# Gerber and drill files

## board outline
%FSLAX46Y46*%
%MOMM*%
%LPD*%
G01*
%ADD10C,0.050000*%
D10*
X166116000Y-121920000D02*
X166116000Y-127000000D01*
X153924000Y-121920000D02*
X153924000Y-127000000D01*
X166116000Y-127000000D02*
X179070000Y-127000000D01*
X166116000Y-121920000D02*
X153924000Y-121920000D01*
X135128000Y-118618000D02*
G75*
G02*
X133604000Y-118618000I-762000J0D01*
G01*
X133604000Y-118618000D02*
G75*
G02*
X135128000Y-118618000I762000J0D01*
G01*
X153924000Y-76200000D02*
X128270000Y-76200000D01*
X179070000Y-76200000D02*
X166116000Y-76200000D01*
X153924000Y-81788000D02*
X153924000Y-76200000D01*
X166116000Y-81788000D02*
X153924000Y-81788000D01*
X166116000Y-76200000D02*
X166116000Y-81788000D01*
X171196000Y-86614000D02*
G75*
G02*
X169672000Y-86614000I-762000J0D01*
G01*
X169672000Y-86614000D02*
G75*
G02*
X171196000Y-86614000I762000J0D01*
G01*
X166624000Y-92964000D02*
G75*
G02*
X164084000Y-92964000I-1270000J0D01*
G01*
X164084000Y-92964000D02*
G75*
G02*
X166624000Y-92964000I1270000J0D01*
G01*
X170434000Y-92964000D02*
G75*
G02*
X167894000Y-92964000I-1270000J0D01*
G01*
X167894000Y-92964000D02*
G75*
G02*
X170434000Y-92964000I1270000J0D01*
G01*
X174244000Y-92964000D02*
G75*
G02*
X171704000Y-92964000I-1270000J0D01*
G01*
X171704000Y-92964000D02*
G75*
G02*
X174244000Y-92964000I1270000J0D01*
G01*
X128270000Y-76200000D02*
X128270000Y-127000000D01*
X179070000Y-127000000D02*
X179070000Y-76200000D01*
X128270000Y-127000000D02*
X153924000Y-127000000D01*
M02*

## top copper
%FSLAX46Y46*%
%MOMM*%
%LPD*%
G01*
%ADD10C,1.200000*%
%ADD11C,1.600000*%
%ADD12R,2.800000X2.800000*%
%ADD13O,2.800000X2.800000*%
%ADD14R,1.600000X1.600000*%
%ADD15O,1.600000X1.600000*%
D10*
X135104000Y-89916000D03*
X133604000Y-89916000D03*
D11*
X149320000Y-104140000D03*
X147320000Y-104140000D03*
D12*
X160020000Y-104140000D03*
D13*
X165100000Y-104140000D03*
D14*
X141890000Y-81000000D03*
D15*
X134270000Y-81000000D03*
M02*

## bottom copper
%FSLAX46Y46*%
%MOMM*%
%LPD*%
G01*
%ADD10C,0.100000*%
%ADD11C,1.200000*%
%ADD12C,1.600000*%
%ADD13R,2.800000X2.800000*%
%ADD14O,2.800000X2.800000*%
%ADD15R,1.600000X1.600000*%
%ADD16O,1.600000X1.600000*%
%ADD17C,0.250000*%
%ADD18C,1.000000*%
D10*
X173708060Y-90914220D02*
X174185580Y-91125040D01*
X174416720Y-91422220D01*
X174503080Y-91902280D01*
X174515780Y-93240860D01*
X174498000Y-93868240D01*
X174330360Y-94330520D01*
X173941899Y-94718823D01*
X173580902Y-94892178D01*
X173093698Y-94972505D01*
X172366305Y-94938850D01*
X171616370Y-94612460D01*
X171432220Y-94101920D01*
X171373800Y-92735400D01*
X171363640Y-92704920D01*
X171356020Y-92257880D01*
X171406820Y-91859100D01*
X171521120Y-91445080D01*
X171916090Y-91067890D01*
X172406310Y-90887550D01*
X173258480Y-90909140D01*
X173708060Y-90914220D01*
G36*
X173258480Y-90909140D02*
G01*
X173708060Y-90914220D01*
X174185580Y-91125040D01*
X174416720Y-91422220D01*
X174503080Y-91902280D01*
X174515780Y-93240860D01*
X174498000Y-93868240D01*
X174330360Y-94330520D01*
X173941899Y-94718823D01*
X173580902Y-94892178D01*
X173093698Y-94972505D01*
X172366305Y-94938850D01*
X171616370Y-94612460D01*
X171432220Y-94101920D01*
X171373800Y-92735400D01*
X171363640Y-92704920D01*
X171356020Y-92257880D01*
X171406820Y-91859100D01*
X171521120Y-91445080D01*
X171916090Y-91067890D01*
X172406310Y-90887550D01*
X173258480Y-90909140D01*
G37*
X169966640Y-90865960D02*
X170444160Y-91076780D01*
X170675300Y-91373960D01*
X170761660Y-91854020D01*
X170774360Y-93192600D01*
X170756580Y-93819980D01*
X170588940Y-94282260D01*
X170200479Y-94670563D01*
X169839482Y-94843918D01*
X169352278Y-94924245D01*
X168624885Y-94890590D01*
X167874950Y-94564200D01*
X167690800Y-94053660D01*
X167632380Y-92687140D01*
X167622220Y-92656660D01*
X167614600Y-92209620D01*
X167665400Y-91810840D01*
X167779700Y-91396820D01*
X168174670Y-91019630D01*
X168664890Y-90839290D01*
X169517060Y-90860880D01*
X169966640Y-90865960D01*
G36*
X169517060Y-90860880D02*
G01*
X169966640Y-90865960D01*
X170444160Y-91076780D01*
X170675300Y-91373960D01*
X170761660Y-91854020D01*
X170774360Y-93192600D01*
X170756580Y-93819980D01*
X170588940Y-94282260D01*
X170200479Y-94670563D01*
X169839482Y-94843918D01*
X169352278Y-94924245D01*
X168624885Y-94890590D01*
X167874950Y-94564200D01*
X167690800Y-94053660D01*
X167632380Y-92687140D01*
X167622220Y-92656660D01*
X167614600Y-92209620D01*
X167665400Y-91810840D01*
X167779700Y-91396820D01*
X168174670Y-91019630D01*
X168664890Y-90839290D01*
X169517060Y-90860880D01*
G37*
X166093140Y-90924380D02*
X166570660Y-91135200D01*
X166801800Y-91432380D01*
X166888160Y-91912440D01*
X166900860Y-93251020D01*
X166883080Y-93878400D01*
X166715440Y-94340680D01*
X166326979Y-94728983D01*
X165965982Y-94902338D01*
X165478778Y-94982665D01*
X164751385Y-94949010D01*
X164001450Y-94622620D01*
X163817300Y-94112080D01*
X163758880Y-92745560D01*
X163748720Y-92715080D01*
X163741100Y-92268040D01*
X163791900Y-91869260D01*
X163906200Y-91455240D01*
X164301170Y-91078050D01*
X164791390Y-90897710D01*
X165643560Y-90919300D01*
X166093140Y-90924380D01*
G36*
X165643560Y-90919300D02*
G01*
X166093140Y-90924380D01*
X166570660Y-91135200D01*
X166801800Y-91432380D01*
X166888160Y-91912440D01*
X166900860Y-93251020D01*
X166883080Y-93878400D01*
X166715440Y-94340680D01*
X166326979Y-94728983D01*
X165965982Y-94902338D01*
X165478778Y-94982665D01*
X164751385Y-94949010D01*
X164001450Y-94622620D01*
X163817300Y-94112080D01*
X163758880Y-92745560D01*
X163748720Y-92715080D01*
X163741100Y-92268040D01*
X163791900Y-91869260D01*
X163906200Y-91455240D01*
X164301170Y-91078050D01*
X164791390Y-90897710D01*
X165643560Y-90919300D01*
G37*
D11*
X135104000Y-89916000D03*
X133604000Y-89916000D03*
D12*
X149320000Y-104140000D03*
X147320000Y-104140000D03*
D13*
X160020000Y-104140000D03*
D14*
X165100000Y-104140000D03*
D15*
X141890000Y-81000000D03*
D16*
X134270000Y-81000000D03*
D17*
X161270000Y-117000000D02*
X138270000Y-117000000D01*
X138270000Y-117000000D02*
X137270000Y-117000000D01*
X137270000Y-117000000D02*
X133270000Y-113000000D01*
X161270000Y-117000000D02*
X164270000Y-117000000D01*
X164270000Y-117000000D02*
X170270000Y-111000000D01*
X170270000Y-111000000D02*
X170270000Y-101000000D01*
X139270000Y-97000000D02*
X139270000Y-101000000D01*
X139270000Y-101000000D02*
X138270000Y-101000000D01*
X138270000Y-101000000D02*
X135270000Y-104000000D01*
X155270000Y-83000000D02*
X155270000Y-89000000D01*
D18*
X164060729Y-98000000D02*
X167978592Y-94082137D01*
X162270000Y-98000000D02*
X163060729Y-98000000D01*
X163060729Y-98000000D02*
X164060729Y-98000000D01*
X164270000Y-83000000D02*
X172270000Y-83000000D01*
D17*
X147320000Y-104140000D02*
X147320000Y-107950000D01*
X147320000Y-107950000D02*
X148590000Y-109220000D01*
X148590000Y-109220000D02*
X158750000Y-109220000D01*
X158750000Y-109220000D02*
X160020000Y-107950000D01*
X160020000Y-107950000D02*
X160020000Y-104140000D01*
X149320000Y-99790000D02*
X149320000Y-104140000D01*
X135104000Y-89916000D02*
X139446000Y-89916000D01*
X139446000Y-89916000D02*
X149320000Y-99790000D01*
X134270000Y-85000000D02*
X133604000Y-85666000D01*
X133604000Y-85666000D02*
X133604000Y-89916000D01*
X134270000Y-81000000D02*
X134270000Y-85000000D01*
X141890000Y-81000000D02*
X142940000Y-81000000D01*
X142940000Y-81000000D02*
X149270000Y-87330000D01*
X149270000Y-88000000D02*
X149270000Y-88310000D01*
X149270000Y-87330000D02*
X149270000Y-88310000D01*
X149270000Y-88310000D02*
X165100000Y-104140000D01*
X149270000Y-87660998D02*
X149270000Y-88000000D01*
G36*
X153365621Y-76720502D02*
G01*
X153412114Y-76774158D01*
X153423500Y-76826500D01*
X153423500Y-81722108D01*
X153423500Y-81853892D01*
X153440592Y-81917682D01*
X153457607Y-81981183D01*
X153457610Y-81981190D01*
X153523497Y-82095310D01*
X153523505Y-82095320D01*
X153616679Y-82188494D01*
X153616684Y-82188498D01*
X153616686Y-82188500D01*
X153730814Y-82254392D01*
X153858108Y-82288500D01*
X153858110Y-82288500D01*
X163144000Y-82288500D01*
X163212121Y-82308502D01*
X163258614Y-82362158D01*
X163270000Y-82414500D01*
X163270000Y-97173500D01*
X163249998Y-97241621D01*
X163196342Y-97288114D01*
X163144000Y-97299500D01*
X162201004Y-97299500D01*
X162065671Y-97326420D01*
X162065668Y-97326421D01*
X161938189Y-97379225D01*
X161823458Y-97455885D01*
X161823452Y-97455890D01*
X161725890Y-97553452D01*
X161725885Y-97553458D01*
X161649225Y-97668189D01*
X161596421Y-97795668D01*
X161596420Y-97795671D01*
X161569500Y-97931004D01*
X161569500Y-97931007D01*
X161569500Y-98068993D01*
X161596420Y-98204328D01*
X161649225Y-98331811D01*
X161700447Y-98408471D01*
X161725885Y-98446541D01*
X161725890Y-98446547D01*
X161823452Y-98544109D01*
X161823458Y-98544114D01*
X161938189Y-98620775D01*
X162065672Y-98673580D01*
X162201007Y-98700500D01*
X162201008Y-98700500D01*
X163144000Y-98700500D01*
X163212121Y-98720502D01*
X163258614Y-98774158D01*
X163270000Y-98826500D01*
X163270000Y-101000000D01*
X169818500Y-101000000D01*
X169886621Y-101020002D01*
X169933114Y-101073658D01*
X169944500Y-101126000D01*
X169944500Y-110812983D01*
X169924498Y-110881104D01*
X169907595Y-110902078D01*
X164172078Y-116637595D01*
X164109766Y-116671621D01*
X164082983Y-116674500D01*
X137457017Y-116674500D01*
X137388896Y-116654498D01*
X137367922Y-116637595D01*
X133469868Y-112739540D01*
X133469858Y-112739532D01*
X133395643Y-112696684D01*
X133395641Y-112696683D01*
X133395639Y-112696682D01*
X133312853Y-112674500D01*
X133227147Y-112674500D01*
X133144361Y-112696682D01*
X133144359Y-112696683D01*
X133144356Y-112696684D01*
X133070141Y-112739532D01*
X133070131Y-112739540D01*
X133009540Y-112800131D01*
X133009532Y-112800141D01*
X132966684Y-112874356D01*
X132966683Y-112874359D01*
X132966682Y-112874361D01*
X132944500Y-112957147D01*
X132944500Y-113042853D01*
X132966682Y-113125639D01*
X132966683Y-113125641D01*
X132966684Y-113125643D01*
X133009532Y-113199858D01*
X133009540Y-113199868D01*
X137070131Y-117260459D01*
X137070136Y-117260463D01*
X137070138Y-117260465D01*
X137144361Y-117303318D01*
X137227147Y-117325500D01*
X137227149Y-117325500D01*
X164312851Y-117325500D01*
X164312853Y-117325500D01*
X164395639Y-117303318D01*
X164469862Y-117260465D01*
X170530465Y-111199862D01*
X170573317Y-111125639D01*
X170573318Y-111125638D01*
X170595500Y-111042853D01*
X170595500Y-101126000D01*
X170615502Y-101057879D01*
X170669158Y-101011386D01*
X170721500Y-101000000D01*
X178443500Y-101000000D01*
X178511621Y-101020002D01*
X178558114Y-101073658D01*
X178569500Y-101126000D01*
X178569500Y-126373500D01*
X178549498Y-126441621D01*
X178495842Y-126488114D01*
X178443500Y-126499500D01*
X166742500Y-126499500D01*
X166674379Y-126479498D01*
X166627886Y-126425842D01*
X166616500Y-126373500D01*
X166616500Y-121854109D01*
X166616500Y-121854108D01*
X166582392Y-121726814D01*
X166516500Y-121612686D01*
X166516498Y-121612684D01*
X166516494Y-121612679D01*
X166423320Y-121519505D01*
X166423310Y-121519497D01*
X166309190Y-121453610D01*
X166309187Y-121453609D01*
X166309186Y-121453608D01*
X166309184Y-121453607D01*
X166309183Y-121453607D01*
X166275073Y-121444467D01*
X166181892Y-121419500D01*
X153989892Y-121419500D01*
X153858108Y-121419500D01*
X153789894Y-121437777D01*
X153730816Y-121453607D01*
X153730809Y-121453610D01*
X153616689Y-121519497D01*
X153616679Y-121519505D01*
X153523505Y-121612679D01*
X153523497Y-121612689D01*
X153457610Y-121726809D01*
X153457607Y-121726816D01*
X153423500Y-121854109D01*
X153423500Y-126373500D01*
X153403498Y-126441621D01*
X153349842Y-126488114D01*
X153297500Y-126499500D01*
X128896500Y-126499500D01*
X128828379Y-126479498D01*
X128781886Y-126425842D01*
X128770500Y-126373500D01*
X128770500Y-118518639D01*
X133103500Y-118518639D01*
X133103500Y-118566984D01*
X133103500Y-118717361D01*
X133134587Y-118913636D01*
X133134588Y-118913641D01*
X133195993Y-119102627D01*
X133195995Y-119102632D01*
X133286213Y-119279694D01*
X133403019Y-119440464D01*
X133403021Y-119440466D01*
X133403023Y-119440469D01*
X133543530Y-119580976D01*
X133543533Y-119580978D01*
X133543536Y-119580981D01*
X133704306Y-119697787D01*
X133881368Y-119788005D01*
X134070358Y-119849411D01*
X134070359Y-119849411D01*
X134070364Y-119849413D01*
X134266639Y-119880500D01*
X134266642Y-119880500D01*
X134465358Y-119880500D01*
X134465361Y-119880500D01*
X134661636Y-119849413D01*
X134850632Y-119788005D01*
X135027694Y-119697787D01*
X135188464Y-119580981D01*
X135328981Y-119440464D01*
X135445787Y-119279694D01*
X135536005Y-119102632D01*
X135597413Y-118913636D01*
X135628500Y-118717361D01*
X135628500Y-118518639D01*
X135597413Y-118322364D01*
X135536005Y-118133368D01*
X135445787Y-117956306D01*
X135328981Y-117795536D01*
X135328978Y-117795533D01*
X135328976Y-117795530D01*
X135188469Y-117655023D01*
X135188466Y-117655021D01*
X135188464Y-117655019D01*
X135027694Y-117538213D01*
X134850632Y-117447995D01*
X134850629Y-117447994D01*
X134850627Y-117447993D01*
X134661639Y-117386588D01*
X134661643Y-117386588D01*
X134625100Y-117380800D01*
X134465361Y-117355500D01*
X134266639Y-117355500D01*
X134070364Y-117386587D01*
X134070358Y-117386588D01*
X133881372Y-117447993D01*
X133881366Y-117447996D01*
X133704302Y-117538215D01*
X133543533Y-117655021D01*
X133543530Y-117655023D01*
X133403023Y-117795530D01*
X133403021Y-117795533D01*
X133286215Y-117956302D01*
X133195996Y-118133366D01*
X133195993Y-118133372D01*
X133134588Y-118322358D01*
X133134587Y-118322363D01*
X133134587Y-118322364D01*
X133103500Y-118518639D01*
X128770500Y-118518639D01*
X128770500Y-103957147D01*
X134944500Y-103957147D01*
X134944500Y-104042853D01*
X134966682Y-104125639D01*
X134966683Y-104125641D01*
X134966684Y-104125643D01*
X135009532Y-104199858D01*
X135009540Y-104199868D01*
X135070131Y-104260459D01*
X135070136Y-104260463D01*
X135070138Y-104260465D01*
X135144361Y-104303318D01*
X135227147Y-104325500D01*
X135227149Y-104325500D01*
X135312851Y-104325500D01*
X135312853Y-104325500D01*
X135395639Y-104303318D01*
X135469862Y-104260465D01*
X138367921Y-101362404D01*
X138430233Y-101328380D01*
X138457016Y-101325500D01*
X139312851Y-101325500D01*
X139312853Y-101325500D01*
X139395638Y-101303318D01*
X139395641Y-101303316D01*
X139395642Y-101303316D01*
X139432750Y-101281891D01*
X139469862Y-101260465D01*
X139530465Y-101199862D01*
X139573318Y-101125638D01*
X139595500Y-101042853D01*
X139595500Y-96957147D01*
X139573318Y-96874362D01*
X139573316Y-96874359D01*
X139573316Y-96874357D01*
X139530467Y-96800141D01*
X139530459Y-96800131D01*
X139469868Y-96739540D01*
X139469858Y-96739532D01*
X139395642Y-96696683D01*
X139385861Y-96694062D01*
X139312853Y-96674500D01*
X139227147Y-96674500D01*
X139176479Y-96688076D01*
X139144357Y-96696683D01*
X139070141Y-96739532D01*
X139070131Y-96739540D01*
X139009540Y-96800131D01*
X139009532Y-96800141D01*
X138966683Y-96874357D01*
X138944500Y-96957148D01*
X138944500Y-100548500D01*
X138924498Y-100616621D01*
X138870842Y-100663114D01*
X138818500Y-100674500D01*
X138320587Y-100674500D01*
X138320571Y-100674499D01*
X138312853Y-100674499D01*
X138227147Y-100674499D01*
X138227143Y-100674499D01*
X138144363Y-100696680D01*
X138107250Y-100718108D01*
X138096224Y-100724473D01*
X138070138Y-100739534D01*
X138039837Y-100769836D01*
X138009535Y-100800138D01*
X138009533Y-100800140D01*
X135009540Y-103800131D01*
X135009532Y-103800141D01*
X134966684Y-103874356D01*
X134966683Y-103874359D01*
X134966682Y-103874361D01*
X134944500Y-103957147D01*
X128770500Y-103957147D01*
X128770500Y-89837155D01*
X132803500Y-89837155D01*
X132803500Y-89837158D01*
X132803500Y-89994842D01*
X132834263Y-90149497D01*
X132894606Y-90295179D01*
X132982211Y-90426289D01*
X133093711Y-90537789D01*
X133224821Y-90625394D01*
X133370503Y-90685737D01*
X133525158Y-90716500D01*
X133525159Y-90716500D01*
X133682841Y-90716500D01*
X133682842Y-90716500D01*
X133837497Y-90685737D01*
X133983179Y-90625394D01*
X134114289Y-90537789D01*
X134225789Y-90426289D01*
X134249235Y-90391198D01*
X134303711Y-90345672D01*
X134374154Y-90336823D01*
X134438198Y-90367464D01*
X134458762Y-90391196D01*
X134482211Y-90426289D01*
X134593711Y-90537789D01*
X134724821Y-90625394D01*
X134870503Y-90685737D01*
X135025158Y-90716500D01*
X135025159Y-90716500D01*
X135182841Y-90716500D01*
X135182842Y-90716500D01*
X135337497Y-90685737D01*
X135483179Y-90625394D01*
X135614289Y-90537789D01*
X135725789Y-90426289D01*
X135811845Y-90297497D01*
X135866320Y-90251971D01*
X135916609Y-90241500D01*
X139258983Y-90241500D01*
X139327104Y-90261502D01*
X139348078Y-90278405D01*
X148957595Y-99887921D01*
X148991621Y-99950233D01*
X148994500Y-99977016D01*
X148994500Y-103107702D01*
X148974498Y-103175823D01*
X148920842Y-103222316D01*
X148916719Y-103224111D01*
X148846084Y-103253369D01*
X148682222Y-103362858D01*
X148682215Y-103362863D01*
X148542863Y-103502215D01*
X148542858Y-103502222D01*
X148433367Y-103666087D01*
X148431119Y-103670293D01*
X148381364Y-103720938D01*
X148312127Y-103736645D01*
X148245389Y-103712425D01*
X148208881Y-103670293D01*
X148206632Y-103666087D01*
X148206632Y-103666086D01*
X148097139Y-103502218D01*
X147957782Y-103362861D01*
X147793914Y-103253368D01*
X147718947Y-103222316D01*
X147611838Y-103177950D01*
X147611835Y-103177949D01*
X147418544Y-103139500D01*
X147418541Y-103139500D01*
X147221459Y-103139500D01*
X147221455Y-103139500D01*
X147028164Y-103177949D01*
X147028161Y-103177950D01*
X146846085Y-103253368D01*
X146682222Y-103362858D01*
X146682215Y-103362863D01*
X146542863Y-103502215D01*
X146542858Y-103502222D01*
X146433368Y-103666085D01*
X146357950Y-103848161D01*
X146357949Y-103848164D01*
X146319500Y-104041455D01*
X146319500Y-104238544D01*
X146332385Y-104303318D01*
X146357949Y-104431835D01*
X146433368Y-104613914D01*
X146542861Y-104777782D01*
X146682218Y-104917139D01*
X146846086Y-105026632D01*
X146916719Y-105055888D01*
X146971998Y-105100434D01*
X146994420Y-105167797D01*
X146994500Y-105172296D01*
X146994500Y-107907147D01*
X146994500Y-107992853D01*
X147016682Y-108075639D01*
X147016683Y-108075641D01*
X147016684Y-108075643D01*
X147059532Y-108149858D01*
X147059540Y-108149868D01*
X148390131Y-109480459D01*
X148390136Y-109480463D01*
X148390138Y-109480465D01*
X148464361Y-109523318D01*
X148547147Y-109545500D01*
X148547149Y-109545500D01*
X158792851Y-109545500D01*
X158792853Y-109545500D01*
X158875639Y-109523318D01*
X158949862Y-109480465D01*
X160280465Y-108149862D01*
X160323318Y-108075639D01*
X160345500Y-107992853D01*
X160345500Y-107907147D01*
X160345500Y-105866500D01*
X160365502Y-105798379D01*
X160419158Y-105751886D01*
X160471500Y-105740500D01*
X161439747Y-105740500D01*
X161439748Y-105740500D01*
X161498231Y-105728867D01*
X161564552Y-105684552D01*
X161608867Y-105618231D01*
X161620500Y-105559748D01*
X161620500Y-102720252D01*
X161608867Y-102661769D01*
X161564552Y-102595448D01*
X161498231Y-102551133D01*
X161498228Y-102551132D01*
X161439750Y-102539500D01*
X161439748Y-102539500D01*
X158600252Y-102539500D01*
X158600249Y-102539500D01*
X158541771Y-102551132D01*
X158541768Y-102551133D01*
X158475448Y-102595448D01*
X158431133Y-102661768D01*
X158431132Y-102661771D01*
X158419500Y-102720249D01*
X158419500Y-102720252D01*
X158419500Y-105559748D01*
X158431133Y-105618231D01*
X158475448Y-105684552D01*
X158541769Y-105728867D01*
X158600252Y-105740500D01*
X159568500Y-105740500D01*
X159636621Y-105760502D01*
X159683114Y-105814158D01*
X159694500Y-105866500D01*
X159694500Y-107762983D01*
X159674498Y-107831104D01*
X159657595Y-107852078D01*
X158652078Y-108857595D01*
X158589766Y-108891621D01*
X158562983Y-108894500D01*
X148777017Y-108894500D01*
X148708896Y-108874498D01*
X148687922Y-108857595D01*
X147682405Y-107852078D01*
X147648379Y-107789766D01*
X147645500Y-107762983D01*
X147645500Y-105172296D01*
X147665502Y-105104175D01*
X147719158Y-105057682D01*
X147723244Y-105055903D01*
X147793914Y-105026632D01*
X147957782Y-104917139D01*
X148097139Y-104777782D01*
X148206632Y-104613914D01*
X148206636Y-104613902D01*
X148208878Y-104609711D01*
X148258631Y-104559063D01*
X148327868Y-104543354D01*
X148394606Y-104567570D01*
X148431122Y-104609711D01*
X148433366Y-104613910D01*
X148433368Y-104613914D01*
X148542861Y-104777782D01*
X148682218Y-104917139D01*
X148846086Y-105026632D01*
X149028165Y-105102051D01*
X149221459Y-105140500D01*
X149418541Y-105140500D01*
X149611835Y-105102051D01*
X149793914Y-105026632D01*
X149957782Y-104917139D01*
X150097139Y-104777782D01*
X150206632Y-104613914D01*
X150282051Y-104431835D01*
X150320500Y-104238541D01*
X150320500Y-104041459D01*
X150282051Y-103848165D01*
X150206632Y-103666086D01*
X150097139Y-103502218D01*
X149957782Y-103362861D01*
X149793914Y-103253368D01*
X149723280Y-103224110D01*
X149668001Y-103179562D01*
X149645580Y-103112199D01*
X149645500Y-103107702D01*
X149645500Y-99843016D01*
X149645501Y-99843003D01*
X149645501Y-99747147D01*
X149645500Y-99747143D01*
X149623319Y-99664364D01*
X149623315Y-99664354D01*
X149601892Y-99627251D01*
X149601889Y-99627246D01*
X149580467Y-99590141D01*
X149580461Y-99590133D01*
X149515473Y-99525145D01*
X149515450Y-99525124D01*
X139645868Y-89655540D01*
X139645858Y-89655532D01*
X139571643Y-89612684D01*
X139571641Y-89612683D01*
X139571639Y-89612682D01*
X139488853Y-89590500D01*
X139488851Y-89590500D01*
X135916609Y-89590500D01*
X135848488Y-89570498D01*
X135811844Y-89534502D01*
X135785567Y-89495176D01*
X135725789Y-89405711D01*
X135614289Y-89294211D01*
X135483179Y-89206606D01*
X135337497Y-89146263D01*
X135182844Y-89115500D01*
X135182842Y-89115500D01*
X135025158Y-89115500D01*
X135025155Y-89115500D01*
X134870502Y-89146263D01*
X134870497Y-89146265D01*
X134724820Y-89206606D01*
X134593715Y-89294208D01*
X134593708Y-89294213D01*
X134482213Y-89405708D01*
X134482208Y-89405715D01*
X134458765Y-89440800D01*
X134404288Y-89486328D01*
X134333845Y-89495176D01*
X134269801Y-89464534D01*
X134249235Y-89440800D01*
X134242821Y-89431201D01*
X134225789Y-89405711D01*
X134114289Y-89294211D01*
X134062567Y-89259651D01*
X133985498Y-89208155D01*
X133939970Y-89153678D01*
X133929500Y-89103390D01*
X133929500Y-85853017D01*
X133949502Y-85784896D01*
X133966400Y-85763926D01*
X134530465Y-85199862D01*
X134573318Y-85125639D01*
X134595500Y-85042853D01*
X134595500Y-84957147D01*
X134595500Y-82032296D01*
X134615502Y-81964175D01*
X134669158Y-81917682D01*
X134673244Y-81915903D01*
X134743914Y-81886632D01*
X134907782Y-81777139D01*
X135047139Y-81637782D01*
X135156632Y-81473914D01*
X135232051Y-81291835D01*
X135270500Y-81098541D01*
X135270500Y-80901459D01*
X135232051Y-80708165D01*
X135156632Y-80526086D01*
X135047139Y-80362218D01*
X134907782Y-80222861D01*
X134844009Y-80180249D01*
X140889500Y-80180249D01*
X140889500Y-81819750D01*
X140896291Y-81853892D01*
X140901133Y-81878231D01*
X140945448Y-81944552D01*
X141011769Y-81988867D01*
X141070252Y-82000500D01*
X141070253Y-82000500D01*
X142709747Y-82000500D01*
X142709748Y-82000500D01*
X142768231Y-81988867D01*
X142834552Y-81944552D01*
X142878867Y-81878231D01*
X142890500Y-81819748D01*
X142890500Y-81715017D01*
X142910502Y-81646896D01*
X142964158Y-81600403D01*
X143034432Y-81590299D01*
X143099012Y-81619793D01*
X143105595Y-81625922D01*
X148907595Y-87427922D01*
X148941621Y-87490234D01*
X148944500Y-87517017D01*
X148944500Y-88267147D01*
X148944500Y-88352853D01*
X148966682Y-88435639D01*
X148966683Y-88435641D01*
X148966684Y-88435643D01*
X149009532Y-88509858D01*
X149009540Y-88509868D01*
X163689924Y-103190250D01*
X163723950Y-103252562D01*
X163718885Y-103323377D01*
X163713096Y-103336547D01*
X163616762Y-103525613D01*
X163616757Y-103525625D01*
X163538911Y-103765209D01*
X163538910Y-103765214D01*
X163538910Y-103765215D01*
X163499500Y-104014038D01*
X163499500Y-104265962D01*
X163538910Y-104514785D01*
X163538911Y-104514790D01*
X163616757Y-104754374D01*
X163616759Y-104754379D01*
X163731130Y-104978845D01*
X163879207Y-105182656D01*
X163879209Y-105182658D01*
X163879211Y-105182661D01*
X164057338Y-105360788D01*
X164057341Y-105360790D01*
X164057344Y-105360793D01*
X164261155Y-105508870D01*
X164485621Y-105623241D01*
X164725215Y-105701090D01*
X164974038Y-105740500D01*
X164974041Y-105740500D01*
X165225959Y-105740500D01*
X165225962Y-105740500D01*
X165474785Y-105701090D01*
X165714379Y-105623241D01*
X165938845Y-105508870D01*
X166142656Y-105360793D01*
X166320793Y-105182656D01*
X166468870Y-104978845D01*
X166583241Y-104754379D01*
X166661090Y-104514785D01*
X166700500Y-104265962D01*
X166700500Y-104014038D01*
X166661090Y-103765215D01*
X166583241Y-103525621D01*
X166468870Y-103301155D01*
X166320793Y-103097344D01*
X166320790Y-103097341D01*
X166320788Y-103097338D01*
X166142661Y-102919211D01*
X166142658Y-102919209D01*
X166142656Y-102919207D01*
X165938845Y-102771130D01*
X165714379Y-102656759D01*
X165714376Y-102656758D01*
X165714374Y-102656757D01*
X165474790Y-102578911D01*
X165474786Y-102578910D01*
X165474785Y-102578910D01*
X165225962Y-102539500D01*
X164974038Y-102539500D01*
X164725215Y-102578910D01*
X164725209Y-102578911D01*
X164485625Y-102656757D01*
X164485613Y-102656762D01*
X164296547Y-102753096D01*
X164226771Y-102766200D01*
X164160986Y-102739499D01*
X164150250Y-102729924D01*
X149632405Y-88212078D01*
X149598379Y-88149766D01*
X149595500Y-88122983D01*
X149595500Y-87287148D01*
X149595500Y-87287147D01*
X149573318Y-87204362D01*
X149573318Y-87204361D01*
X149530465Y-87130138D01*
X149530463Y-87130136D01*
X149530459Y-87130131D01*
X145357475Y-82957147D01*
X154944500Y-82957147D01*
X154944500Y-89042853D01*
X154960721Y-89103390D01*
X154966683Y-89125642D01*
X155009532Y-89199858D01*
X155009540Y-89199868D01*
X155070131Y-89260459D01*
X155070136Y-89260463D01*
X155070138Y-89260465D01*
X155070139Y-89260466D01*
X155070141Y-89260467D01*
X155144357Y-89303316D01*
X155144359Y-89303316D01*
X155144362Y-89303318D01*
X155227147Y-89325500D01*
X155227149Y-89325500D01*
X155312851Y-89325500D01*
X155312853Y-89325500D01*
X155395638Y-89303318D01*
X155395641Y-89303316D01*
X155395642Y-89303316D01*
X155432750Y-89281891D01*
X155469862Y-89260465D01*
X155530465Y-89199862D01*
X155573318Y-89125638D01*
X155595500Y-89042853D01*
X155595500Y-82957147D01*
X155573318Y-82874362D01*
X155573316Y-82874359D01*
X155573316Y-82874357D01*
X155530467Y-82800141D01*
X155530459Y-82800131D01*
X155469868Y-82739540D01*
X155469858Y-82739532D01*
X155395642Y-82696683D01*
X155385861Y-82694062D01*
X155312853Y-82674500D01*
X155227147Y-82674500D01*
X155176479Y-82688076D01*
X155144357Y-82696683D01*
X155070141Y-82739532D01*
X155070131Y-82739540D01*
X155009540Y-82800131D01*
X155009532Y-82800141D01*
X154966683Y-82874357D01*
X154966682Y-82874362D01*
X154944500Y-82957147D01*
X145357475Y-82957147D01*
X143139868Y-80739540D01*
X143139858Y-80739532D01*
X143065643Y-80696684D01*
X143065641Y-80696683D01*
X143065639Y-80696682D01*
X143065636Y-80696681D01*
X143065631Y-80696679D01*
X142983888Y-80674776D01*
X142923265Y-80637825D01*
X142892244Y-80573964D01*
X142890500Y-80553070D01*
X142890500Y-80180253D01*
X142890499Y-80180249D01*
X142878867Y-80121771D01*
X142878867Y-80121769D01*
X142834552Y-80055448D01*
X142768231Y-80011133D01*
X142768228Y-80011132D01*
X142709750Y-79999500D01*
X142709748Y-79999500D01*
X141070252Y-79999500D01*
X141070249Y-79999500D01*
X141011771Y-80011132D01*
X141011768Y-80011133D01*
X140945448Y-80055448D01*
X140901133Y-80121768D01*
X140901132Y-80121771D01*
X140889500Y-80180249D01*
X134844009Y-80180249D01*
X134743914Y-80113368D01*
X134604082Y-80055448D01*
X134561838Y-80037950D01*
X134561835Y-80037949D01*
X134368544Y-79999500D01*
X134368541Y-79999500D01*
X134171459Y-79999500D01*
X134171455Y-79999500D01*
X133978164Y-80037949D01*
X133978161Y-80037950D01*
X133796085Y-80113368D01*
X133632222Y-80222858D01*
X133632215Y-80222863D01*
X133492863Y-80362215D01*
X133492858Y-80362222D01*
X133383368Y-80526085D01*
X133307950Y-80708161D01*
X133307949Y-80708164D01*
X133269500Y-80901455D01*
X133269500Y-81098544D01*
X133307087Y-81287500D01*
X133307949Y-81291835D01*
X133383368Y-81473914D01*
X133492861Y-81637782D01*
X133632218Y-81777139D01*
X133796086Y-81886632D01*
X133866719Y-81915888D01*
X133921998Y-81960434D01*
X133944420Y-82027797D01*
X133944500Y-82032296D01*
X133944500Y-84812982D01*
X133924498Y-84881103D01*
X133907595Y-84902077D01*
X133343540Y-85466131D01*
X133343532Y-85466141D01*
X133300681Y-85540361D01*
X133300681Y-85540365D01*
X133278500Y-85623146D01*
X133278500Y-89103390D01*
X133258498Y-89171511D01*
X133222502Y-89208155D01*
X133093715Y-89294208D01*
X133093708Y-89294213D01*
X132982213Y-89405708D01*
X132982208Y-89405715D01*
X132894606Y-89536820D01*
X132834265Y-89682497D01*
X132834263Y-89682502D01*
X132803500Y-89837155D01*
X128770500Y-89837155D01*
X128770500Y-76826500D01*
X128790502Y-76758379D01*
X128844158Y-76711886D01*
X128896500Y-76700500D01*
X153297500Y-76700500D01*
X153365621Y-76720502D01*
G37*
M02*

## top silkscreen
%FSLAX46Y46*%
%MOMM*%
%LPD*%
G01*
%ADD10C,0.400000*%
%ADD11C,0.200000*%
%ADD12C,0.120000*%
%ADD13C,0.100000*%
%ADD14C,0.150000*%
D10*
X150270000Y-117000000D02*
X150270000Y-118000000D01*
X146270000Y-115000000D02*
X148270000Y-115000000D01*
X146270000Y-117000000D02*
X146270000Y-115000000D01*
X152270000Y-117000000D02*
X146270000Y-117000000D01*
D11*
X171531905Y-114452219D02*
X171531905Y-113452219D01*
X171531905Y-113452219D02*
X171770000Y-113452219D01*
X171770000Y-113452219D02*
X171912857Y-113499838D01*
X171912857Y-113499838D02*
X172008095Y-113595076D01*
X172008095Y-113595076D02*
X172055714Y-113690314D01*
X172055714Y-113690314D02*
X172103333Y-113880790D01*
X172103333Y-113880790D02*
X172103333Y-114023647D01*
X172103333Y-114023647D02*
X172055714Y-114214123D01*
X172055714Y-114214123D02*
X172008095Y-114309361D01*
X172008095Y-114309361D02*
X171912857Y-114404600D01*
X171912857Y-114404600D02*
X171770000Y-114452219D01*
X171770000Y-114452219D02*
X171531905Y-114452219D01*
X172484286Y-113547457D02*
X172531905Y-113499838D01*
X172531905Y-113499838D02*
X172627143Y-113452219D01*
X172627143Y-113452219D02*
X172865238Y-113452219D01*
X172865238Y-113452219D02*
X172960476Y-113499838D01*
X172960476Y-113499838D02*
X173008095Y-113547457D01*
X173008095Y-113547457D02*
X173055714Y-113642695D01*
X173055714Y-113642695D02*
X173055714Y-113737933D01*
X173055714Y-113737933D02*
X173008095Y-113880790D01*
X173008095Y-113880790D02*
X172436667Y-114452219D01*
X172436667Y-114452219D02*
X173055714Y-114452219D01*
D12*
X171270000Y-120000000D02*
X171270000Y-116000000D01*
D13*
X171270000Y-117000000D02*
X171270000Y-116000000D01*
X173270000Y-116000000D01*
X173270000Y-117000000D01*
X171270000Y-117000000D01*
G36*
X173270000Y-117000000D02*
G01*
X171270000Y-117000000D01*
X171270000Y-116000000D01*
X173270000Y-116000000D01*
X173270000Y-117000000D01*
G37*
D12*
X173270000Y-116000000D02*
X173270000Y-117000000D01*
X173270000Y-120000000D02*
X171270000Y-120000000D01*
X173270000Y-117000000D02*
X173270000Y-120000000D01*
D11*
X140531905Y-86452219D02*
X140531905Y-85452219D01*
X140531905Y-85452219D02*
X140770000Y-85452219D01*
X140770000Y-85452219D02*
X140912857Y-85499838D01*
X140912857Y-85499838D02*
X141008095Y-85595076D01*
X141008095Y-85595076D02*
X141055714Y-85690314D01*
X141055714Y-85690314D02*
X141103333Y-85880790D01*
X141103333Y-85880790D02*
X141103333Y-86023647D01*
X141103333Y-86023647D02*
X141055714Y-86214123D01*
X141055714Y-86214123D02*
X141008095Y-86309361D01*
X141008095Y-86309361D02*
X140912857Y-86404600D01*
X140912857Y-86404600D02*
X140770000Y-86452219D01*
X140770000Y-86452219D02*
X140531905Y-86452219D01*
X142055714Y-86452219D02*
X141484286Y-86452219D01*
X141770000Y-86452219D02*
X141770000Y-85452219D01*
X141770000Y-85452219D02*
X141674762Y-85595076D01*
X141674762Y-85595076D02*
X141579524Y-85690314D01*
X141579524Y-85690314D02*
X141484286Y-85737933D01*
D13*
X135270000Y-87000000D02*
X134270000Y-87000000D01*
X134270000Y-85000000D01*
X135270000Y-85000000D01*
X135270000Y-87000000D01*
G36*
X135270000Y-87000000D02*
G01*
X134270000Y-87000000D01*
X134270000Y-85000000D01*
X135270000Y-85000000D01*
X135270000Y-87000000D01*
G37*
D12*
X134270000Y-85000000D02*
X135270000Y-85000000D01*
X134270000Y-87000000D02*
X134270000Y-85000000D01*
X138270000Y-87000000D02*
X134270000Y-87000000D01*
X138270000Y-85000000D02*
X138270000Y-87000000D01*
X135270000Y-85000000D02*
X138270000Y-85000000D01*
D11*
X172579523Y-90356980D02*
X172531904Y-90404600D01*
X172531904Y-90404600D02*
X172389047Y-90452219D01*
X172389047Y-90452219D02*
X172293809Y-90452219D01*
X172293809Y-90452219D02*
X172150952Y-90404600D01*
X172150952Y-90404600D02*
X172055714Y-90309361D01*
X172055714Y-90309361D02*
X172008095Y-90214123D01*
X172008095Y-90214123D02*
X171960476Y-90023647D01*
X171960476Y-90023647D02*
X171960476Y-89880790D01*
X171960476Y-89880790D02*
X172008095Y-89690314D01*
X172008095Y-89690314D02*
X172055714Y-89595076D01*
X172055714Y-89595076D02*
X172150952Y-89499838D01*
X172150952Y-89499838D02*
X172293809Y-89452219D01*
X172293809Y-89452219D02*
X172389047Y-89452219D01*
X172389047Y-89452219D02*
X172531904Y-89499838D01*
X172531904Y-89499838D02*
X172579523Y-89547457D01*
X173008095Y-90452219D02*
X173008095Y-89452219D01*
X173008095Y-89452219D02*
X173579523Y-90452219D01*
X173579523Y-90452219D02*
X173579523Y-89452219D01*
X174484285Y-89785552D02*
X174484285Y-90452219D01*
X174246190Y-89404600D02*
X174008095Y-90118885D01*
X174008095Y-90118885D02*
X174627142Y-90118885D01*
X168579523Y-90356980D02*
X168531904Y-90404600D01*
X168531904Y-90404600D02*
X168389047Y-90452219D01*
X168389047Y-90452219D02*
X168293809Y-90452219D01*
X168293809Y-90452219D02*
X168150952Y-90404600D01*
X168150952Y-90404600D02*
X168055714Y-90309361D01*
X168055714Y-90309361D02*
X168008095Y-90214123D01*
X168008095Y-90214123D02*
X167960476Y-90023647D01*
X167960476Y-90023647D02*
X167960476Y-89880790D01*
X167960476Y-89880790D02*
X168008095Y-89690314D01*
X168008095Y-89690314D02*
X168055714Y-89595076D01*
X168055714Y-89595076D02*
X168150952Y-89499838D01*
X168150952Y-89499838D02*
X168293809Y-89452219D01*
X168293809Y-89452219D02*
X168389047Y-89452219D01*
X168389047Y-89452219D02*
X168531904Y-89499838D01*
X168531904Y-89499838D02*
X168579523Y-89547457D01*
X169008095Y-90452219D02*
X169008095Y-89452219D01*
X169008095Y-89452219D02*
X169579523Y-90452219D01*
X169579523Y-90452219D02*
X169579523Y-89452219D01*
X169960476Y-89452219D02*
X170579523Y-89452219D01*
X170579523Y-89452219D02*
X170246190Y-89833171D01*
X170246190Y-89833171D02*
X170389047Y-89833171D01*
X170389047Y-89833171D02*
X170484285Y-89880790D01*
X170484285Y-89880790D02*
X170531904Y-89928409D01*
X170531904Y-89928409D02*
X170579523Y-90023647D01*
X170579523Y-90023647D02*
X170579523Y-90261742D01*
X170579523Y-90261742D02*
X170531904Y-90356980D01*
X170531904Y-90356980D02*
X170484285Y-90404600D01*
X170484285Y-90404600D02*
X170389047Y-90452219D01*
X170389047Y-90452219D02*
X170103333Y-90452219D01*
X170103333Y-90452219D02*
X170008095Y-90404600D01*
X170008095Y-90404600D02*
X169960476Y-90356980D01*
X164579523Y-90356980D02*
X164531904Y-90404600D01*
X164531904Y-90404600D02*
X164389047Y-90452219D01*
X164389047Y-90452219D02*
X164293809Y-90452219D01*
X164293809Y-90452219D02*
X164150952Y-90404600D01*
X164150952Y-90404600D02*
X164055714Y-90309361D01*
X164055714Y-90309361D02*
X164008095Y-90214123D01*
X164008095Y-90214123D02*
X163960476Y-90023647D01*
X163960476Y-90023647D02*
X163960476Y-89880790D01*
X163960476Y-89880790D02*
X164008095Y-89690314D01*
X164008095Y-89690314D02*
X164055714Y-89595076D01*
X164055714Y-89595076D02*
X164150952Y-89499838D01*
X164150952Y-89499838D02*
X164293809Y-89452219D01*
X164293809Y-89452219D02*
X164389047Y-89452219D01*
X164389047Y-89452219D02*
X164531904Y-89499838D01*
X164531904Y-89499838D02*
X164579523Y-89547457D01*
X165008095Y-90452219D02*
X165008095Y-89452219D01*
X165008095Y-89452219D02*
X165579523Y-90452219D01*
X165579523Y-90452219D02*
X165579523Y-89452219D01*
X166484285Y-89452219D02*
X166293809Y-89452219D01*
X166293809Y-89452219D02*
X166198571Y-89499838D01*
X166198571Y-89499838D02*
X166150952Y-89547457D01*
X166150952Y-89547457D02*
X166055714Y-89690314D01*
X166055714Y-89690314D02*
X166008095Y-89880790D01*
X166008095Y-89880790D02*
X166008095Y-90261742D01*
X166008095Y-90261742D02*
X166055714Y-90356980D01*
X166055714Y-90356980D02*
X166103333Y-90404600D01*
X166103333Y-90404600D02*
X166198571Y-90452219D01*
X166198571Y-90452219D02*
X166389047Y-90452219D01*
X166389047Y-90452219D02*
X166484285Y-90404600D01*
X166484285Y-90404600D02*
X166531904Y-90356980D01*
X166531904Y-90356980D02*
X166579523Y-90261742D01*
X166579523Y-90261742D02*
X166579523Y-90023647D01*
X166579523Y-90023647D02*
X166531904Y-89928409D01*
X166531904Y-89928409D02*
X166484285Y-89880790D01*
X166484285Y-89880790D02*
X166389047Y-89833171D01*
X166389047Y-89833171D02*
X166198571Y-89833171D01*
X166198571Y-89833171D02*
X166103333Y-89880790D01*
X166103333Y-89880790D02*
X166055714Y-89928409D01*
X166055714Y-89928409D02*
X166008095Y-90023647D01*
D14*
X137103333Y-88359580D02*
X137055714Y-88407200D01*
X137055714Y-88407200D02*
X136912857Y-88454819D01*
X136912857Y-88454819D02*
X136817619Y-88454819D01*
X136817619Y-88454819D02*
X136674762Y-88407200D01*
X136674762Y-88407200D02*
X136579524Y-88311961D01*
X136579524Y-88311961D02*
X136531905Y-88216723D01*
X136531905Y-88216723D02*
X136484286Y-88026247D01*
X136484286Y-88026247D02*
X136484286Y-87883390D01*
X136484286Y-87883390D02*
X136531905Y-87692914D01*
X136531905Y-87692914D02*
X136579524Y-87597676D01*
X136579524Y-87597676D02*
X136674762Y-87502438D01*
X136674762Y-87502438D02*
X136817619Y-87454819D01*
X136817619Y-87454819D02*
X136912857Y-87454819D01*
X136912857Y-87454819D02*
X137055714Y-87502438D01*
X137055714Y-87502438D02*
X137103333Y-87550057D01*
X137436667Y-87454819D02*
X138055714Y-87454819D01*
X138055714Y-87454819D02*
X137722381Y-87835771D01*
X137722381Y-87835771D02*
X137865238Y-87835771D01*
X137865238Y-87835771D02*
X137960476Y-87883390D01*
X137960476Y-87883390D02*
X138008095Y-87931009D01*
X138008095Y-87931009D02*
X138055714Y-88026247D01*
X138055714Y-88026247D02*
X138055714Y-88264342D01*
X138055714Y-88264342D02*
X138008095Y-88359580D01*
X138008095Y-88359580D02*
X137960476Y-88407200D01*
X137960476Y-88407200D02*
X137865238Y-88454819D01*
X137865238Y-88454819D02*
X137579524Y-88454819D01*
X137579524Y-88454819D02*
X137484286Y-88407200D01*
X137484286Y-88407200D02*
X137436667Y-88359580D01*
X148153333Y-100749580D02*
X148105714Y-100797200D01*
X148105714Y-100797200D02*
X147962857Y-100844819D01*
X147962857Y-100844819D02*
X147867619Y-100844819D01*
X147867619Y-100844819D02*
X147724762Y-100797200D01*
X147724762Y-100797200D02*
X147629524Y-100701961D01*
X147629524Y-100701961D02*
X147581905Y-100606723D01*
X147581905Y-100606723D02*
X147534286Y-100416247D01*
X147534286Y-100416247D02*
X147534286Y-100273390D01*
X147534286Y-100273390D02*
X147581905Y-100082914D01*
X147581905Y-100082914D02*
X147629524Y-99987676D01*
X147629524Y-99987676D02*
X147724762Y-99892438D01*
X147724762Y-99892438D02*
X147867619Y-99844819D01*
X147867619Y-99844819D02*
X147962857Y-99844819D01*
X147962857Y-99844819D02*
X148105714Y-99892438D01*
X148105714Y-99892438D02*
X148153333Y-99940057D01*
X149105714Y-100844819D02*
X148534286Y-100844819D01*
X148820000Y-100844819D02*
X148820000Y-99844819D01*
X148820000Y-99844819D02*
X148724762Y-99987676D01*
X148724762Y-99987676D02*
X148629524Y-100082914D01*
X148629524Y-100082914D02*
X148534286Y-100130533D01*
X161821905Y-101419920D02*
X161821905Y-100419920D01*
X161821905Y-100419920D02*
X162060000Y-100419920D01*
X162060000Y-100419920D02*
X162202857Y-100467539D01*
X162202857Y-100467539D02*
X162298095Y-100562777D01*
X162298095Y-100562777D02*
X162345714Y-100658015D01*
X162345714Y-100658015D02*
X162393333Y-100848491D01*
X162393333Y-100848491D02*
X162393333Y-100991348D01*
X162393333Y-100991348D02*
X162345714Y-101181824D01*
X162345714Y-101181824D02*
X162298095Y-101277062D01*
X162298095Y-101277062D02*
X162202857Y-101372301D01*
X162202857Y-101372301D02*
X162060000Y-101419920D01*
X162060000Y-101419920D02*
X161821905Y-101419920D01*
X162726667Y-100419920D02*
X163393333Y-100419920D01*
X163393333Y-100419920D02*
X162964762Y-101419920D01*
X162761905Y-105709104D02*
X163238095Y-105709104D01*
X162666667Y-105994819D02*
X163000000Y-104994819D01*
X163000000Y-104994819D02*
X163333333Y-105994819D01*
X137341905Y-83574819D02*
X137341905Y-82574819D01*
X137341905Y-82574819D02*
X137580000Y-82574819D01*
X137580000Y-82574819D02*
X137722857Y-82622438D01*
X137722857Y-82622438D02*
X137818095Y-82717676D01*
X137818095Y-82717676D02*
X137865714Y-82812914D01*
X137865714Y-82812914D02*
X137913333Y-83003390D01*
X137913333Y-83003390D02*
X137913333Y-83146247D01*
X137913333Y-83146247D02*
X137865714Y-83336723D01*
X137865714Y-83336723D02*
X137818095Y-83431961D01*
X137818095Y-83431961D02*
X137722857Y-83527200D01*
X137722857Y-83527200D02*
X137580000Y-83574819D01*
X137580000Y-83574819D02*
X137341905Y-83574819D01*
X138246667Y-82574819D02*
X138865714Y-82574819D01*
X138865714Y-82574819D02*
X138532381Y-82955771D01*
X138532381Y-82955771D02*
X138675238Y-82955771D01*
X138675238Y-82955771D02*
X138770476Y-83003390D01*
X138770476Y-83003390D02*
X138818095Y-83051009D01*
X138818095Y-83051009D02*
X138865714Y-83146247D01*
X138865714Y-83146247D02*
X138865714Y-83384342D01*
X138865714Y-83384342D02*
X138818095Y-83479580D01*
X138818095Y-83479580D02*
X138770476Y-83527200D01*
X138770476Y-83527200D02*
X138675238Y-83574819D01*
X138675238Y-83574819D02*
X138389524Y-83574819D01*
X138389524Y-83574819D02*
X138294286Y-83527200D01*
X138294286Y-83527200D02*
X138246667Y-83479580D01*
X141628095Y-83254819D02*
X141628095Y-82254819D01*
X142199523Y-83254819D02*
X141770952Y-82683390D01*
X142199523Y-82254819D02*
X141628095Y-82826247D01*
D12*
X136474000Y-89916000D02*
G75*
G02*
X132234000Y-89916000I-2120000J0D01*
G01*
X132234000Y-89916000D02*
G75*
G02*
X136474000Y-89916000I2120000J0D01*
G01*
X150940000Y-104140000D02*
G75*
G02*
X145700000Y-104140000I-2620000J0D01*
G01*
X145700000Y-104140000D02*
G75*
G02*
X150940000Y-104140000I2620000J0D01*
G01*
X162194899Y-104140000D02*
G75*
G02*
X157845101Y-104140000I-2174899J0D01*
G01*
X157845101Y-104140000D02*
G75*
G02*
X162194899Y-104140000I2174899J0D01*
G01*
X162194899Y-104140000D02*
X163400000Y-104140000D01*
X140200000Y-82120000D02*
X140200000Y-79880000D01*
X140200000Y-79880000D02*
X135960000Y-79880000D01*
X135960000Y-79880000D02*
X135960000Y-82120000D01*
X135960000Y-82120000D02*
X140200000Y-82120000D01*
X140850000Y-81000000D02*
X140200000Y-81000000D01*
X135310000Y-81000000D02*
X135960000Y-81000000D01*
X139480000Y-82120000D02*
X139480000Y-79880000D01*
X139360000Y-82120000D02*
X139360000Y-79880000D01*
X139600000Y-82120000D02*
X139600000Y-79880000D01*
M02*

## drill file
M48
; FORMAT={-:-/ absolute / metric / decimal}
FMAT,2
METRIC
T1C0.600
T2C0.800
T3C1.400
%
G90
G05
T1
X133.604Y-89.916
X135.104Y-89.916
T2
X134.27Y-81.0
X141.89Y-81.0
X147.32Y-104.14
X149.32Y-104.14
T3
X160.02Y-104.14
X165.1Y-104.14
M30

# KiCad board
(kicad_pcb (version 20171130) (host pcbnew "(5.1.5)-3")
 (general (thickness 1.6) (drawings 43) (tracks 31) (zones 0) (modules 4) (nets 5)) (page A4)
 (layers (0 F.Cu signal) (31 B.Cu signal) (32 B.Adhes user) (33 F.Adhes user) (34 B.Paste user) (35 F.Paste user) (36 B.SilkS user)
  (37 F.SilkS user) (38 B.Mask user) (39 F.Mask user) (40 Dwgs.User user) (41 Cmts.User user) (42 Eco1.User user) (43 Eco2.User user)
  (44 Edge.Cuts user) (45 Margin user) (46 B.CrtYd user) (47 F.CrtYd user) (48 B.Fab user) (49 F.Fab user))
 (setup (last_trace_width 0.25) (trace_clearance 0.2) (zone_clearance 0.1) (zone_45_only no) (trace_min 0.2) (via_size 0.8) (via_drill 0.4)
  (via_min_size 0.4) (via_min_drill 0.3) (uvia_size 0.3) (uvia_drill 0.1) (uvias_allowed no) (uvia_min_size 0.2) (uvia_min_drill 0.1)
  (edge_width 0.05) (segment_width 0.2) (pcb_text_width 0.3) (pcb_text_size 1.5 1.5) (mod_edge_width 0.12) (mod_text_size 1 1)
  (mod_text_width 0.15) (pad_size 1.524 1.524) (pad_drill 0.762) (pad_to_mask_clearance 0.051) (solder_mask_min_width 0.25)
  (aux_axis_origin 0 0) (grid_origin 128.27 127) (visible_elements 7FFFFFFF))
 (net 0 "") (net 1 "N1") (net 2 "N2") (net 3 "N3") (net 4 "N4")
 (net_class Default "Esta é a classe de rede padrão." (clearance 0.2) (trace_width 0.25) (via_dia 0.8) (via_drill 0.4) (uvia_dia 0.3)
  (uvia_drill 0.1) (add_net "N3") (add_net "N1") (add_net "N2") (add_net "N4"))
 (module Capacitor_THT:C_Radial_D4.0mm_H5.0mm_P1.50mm (layer F.Cu) (at 133.604 89.916)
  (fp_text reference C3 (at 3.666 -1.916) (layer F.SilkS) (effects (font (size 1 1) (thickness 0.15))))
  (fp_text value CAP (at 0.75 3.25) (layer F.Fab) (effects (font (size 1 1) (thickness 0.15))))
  (fp_circle (center 0.75 0) (end 2.87 0) (layer F.SilkS) (width 0.12))
  (pad 2 thru_hole circle (at 1.5 0) (size 1.2 1.2) (drill 0.6) (layers *.Cu *.Mask) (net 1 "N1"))
  (pad 1 thru_hole circle (at 0 0) (size 1.2 1.2) (drill 0.6) (layers *.Cu *.Mask) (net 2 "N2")))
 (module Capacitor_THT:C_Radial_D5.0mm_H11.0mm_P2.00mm (layer F.Cu) (at 147.32 104.14)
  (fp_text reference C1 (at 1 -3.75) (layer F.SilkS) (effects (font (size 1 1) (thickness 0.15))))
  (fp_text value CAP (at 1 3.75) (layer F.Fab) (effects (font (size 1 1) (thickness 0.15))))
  (fp_circle (center 1 0) (end 3.62 0) (layer F.SilkS) (width 0.12))
  (pad 2 thru_hole circle (at 2 0) (size 1.6 1.6) (drill 0.8) (layers *.Cu *.Mask) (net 1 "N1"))
  (pad 1 thru_hole circle (at 0 0) (size 1.6 1.6) (drill 0.8) (layers *.Cu *.Mask) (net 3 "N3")))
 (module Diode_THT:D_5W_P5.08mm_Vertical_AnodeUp (layer F.Cu) (at 160.02 104.14)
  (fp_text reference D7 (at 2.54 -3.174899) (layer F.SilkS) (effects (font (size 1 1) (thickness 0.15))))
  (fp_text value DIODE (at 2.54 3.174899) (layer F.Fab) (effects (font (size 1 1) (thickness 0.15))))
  (fp_circle (center 0 0) (end 2.174899 0) (layer F.SilkS) (width 0.12))
  (fp_line (start 2.174899 0) (end 3.38 0) (layer F.SilkS) (width 0.12))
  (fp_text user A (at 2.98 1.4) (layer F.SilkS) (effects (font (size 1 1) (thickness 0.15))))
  (pad 1 thru_hole rect (at 0 0) (size 2.8 2.8) (drill 1.4) (layers *.Cu *.Mask) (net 3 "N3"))
  (pad 2 thru_hole oval (at 5.08 0) (size 2.8 2.8) (drill 1.4) (layers *.Cu *.Mask) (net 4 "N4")))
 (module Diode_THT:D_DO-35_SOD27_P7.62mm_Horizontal (layer F.Cu) (at 141.89 81 180)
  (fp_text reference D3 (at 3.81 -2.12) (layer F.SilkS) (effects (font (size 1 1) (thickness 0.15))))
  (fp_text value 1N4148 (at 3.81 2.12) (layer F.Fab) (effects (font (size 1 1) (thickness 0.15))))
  (fp_line (start 1.69 -1.12) (end 1.69 1.12) (layer F.SilkS) (width 0.12))
  (fp_line (start 1.69 1.12) (end 5.93 1.12) (layer F.SilkS) (width 0.12))
  (fp_line (start 5.93 1.12) (end 5.93 -1.12) (layer F.SilkS) (width 0.12))
  (fp_line (start 5.93 -1.12) (end 1.69 -1.12) (layer F.SilkS) (width 0.12))
  (fp_line (start 1.04 0) (end 1.69 0) (layer F.SilkS) (width 0.12))
  (fp_line (start 6.58 0) (end 5.93 0) (layer F.SilkS) (width 0.12))
  (fp_line (start 2.41 -1.12) (end 2.41 1.12) (layer F.SilkS) (width 0.12))
  (fp_line (start 2.53 -1.12) (end 2.53 1.12) (layer F.SilkS) (width 0.12))
  (fp_line (start 2.29 -1.12) (end 2.29 1.12) (layer F.SilkS) (width 0.12))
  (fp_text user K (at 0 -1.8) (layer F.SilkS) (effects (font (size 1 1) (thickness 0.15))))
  (pad 1 thru_hole rect (at 0 0 180) (size 1.6 1.6) (drill 0.8) (layers *.Cu *.Mask) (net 4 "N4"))
  (pad 2 thru_hole oval (at 7.62 0 180) (size 1.6 1.6) (drill 0.8) (layers *.Cu *.Mask) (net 2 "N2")))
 (gr_poly
  (pts (xy 173.70806 90.91422) (xy 174.18558 91.12504) (xy 174.41672 91.42222) (xy 174.50308 91.90228) (xy 174.51578 93.24086)
   (xy 174.498 93.86824) (xy 174.33036 94.33052) (xy 173.941899 94.718823) (xy 173.580902 94.892178) (xy 173.093698 94.972505)
   (xy 172.366305 94.93885) (xy 171.61637 94.61246) (xy 171.43222 94.10192) (xy 171.3738 92.7354) (xy 171.36364 92.70492)
   (xy 171.35602 92.25788) (xy 171.40682 91.8591) (xy 171.52112 91.44508) (xy 171.91609 91.06789) (xy 172.40631 90.88755)
   (xy 173.25848 90.90914))
  (layer B.Cu) (width 0.1))
 (gr_poly
  (pts (xy 169.96664 90.86596) (xy 170.44416 91.07678) (xy 170.6753 91.37396) (xy 170.76166 91.85402) (xy 170.77436 93.1926)
   (xy 170.75658 93.81998) (xy 170.58894 94.28226) (xy 170.200479 94.670563) (xy 169.839482 94.843918) (xy 169.352278 94.924245)
   (xy 168.624885 94.89059) (xy 167.87495 94.5642) (xy 167.6908 94.05366) (xy 167.63238 92.68714) (xy 167.62222 92.65666)
   (xy 167.6146 92.20962) (xy 167.6654 91.81084) (xy 167.7797 91.39682) (xy 168.17467 91.01963) (xy 168.66489 90.83929)
   (xy 169.51706 90.86088))
  (layer B.Cu) (width 0.1))
 (gr_poly
  (pts (xy 166.09314 90.92438) (xy 166.57066 91.1352) (xy 166.8018 91.43238) (xy 166.88816 91.91244) (xy 166.90086 93.25102)
   (xy 166.88308 93.8784) (xy 166.71544 94.34068) (xy 166.326979 94.728983) (xy 165.965982 94.902338) (xy 165.478778 94.982665)
   (xy 164.751385 94.94901) (xy 164.00145 94.62262) (xy 163.8173 94.11208) (xy 163.75888 92.74556) (xy 163.74872 92.71508)
   (xy 163.7411 92.26804) (xy 163.7919 91.86926) (xy 163.9062 91.45524) (xy 164.30117 91.07805) (xy 164.79139 90.89771)
   (xy 165.64356 90.9193))
  (layer B.Cu) (width 0.1))
 (gr_line (start 150.27 117) (end 150.27 118) (layer F.SilkS) (width 0.4))
 (gr_line (start 146.27 115) (end 148.27 115) (layer F.SilkS) (width 0.4))
 (gr_line (start 146.27 117) (end 146.27 115) (layer F.SilkS) (width 0.4))
 (gr_line (start 152.27 117) (end 146.27 117) (layer F.SilkS) (width 0.4))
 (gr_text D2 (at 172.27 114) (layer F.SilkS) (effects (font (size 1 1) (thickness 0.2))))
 (gr_line (start 171.27 120) (end 171.27 116) (layer F.SilkS) (width 0.12))
 (gr_poly (pts (xy 171.27 117) (xy 171.27 116) (xy 173.27 116) (xy 173.27 117)) (layer F.SilkS) (width 0.1))
 (gr_line (start 173.27 116) (end 173.27 117) (layer F.SilkS) (width 0.12))
 (gr_line (start 173.27 120) (end 171.27 120) (layer F.SilkS) (width 0.12))
 (gr_line (start 173.27 117) (end 173.27 120) (layer F.SilkS) (width 0.12))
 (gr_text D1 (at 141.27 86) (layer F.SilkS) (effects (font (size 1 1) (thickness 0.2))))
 (gr_poly (pts (xy 135.27 87) (xy 134.27 87) (xy 134.27 85) (xy 135.27 85)) (layer F.SilkS) (width 0.1))
 (gr_line (start 134.27 85) (end 135.27 85) (layer F.SilkS) (width 0.12))
 (gr_line (start 134.27 87) (end 134.27 85) (layer F.SilkS) (width 0.12))
 (gr_line (start 138.27 87) (end 134.27 87) (layer F.SilkS) (width 0.12))
 (gr_line (start 138.27 85) (end 138.27 87) (layer F.SilkS) (width 0.12))
 (gr_line (start 135.27 85) (end 138.27 85) (layer F.SilkS) (width 0.12))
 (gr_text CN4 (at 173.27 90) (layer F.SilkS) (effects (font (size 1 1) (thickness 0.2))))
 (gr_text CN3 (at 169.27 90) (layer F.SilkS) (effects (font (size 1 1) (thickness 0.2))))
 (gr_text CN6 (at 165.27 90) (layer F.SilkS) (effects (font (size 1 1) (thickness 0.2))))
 (gr_line (start 166.116 121.92) (end 166.116 127) (layer Edge.Cuts) (width 0.05))
 (gr_line (start 153.924 121.92) (end 153.924 127) (layer Edge.Cuts) (width 0.05))
 (gr_line (start 166.116 127) (end 179.07 127) (layer Edge.Cuts) (width 0.05))
 (gr_line (start 166.116 121.92) (end 153.924 121.92) (layer Edge.Cuts) (width 0.05))
 (gr_circle (center 134.366 118.618) (end 135.128 118.618) (layer Edge.Cuts) (width 0.05))
 (gr_line (start 153.924 76.2) (end 128.27 76.2) (layer Edge.Cuts) (width 0.05))
 (gr_line (start 179.07 76.2) (end 166.116 76.2) (layer Edge.Cuts) (width 0.05))
 (gr_line (start 153.924 81.788) (end 153.924 76.2) (layer Edge.Cuts) (width 0.05))
 (gr_line (start 166.116 81.788) (end 153.924 81.788) (layer Edge.Cuts) (width 0.05))
 (gr_line (start 166.116 76.2) (end 166.116 81.788) (layer Edge.Cuts) (width 0.05))
 (gr_circle (center 170.434 86.614) (end 171.196 86.614) (layer Edge.Cuts) (width 0.05))
 (gr_circle (center 165.354 92.964) (end 166.624 92.964) (layer Edge.Cuts) (width 0.05))
 (gr_circle (center 169.164 92.964) (end 170.434 92.964) (layer Edge.Cuts) (width 0.05))
 (gr_circle (center 172.974 92.964) (end 174.244 92.964) (layer Edge.Cuts) (width 0.05))
 (gr_line (start 128.27 76.2) (end 128.27 127) (layer Edge.Cuts) (width 0.05))
 (gr_line (start 179.07 127) (end 179.07 76.2) (layer Edge.Cuts) (width 0.05))
 (gr_line (start 128.27 127) (end 153.924 127) (layer Edge.Cuts) (width 0.05))
 (segment (start 161.27 117) (end 138.27 117) (width 0.25) (layer B.Cu) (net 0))
 (segment (start 138.27 117) (end 137.27 117) (width 0.25) (layer B.Cu) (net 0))
 (segment (start 137.27 117) (end 133.27 113) (width 0.25) (layer B.Cu) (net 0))
 (segment (start 161.27 117) (end 164.27 117) (width 0.25) (layer B.Cu) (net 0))
 (segment (start 164.27 117) (end 170.27 111) (width 0.25) (layer B.Cu) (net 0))
 (segment (start 170.27 111) (end 170.27 101) (width 0.25) (layer B.Cu) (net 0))
 (segment (start 139.27 97) (end 139.27 101) (width 0.25) (layer B.Cu) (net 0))
 (segment (start 139.27 101) (end 138.27 101) (width 0.25) (layer B.Cu) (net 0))
 (segment (start 138.27 101) (end 135.27 104) (width 0.25) (layer B.Cu) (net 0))
 (segment (start 155.27 83) (end 155.27 89) (width 0.25) (layer B.Cu) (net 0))
 (segment (start 164.060729 98) (end 167.978592 94.082137) (width 1) (layer B.Cu) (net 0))
 (segment (start 162.27 98) (end 163.060729 98) (width 1) (layer B.Cu) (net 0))
 (segment (start 163.060729 98) (end 164.060729 98) (width 1) (layer B.Cu) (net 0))
 (segment (start 164.27 83) (end 172.27 83) (width 1) (layer B.Cu) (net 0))
 (segment (start 147.32 104.14) (end 147.32 107.95) (width 0.25) (layer B.Cu) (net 3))
 (segment (start 147.32 107.95) (end 148.59 109.22) (width 0.25) (layer B.Cu) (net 3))
 (segment (start 148.59 109.22) (end 158.75 109.22) (width 0.25) (layer B.Cu) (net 3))
 (segment (start 158.75 109.22) (end 160.02 107.95) (width 0.25) (layer B.Cu) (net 3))
 (segment (start 160.02 107.95) (end 160.02 104.14) (width 0.25) (layer B.Cu) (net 3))
 (segment (start 149.32 99.79) (end 149.32 104.14) (width 0.25) (layer B.Cu) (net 1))
 (segment (start 135.104 89.916) (end 139.446 89.916) (width 0.25) (layer B.Cu) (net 1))
 (segment (start 139.446 89.916) (end 149.32 99.79) (width 0.25) (layer B.Cu) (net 1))
 (segment (start 134.27 85) (end 133.604 85.666) (width 0.25) (layer B.Cu) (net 2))
 (segment (start 133.604 85.666) (end 133.604 89.916) (width 0.25) (layer B.Cu) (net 2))
 (segment (start 134.27 81) (end 134.27 85) (width 0.25) (layer B.Cu) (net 2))
 (segment (start 141.89 81) (end 142.94 81) (width 0.25) (layer B.Cu) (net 4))
 (segment (start 142.94 81) (end 149.27 87.33) (width 0.25) (layer B.Cu) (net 4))
 (segment (start 149.27 88) (end 149.27 88.31) (width 0.25) (layer B.Cu) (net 4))
 (segment (start 149.27 87.33) (end 149.27 88.31) (width 0.25) (layer B.Cu) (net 4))
 (segment (start 149.27 88.31) (end 165.1 104.14) (width 0.25) (layer B.Cu) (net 4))
 (segment (start 149.27 87.660998) (end 149.27 88) (width 0.25) (layer B.Cu) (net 4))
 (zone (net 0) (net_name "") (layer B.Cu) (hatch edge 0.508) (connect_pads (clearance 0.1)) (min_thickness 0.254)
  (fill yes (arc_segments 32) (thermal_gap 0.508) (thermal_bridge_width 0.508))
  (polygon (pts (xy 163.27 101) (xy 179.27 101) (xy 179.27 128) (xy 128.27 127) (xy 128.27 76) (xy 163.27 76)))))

